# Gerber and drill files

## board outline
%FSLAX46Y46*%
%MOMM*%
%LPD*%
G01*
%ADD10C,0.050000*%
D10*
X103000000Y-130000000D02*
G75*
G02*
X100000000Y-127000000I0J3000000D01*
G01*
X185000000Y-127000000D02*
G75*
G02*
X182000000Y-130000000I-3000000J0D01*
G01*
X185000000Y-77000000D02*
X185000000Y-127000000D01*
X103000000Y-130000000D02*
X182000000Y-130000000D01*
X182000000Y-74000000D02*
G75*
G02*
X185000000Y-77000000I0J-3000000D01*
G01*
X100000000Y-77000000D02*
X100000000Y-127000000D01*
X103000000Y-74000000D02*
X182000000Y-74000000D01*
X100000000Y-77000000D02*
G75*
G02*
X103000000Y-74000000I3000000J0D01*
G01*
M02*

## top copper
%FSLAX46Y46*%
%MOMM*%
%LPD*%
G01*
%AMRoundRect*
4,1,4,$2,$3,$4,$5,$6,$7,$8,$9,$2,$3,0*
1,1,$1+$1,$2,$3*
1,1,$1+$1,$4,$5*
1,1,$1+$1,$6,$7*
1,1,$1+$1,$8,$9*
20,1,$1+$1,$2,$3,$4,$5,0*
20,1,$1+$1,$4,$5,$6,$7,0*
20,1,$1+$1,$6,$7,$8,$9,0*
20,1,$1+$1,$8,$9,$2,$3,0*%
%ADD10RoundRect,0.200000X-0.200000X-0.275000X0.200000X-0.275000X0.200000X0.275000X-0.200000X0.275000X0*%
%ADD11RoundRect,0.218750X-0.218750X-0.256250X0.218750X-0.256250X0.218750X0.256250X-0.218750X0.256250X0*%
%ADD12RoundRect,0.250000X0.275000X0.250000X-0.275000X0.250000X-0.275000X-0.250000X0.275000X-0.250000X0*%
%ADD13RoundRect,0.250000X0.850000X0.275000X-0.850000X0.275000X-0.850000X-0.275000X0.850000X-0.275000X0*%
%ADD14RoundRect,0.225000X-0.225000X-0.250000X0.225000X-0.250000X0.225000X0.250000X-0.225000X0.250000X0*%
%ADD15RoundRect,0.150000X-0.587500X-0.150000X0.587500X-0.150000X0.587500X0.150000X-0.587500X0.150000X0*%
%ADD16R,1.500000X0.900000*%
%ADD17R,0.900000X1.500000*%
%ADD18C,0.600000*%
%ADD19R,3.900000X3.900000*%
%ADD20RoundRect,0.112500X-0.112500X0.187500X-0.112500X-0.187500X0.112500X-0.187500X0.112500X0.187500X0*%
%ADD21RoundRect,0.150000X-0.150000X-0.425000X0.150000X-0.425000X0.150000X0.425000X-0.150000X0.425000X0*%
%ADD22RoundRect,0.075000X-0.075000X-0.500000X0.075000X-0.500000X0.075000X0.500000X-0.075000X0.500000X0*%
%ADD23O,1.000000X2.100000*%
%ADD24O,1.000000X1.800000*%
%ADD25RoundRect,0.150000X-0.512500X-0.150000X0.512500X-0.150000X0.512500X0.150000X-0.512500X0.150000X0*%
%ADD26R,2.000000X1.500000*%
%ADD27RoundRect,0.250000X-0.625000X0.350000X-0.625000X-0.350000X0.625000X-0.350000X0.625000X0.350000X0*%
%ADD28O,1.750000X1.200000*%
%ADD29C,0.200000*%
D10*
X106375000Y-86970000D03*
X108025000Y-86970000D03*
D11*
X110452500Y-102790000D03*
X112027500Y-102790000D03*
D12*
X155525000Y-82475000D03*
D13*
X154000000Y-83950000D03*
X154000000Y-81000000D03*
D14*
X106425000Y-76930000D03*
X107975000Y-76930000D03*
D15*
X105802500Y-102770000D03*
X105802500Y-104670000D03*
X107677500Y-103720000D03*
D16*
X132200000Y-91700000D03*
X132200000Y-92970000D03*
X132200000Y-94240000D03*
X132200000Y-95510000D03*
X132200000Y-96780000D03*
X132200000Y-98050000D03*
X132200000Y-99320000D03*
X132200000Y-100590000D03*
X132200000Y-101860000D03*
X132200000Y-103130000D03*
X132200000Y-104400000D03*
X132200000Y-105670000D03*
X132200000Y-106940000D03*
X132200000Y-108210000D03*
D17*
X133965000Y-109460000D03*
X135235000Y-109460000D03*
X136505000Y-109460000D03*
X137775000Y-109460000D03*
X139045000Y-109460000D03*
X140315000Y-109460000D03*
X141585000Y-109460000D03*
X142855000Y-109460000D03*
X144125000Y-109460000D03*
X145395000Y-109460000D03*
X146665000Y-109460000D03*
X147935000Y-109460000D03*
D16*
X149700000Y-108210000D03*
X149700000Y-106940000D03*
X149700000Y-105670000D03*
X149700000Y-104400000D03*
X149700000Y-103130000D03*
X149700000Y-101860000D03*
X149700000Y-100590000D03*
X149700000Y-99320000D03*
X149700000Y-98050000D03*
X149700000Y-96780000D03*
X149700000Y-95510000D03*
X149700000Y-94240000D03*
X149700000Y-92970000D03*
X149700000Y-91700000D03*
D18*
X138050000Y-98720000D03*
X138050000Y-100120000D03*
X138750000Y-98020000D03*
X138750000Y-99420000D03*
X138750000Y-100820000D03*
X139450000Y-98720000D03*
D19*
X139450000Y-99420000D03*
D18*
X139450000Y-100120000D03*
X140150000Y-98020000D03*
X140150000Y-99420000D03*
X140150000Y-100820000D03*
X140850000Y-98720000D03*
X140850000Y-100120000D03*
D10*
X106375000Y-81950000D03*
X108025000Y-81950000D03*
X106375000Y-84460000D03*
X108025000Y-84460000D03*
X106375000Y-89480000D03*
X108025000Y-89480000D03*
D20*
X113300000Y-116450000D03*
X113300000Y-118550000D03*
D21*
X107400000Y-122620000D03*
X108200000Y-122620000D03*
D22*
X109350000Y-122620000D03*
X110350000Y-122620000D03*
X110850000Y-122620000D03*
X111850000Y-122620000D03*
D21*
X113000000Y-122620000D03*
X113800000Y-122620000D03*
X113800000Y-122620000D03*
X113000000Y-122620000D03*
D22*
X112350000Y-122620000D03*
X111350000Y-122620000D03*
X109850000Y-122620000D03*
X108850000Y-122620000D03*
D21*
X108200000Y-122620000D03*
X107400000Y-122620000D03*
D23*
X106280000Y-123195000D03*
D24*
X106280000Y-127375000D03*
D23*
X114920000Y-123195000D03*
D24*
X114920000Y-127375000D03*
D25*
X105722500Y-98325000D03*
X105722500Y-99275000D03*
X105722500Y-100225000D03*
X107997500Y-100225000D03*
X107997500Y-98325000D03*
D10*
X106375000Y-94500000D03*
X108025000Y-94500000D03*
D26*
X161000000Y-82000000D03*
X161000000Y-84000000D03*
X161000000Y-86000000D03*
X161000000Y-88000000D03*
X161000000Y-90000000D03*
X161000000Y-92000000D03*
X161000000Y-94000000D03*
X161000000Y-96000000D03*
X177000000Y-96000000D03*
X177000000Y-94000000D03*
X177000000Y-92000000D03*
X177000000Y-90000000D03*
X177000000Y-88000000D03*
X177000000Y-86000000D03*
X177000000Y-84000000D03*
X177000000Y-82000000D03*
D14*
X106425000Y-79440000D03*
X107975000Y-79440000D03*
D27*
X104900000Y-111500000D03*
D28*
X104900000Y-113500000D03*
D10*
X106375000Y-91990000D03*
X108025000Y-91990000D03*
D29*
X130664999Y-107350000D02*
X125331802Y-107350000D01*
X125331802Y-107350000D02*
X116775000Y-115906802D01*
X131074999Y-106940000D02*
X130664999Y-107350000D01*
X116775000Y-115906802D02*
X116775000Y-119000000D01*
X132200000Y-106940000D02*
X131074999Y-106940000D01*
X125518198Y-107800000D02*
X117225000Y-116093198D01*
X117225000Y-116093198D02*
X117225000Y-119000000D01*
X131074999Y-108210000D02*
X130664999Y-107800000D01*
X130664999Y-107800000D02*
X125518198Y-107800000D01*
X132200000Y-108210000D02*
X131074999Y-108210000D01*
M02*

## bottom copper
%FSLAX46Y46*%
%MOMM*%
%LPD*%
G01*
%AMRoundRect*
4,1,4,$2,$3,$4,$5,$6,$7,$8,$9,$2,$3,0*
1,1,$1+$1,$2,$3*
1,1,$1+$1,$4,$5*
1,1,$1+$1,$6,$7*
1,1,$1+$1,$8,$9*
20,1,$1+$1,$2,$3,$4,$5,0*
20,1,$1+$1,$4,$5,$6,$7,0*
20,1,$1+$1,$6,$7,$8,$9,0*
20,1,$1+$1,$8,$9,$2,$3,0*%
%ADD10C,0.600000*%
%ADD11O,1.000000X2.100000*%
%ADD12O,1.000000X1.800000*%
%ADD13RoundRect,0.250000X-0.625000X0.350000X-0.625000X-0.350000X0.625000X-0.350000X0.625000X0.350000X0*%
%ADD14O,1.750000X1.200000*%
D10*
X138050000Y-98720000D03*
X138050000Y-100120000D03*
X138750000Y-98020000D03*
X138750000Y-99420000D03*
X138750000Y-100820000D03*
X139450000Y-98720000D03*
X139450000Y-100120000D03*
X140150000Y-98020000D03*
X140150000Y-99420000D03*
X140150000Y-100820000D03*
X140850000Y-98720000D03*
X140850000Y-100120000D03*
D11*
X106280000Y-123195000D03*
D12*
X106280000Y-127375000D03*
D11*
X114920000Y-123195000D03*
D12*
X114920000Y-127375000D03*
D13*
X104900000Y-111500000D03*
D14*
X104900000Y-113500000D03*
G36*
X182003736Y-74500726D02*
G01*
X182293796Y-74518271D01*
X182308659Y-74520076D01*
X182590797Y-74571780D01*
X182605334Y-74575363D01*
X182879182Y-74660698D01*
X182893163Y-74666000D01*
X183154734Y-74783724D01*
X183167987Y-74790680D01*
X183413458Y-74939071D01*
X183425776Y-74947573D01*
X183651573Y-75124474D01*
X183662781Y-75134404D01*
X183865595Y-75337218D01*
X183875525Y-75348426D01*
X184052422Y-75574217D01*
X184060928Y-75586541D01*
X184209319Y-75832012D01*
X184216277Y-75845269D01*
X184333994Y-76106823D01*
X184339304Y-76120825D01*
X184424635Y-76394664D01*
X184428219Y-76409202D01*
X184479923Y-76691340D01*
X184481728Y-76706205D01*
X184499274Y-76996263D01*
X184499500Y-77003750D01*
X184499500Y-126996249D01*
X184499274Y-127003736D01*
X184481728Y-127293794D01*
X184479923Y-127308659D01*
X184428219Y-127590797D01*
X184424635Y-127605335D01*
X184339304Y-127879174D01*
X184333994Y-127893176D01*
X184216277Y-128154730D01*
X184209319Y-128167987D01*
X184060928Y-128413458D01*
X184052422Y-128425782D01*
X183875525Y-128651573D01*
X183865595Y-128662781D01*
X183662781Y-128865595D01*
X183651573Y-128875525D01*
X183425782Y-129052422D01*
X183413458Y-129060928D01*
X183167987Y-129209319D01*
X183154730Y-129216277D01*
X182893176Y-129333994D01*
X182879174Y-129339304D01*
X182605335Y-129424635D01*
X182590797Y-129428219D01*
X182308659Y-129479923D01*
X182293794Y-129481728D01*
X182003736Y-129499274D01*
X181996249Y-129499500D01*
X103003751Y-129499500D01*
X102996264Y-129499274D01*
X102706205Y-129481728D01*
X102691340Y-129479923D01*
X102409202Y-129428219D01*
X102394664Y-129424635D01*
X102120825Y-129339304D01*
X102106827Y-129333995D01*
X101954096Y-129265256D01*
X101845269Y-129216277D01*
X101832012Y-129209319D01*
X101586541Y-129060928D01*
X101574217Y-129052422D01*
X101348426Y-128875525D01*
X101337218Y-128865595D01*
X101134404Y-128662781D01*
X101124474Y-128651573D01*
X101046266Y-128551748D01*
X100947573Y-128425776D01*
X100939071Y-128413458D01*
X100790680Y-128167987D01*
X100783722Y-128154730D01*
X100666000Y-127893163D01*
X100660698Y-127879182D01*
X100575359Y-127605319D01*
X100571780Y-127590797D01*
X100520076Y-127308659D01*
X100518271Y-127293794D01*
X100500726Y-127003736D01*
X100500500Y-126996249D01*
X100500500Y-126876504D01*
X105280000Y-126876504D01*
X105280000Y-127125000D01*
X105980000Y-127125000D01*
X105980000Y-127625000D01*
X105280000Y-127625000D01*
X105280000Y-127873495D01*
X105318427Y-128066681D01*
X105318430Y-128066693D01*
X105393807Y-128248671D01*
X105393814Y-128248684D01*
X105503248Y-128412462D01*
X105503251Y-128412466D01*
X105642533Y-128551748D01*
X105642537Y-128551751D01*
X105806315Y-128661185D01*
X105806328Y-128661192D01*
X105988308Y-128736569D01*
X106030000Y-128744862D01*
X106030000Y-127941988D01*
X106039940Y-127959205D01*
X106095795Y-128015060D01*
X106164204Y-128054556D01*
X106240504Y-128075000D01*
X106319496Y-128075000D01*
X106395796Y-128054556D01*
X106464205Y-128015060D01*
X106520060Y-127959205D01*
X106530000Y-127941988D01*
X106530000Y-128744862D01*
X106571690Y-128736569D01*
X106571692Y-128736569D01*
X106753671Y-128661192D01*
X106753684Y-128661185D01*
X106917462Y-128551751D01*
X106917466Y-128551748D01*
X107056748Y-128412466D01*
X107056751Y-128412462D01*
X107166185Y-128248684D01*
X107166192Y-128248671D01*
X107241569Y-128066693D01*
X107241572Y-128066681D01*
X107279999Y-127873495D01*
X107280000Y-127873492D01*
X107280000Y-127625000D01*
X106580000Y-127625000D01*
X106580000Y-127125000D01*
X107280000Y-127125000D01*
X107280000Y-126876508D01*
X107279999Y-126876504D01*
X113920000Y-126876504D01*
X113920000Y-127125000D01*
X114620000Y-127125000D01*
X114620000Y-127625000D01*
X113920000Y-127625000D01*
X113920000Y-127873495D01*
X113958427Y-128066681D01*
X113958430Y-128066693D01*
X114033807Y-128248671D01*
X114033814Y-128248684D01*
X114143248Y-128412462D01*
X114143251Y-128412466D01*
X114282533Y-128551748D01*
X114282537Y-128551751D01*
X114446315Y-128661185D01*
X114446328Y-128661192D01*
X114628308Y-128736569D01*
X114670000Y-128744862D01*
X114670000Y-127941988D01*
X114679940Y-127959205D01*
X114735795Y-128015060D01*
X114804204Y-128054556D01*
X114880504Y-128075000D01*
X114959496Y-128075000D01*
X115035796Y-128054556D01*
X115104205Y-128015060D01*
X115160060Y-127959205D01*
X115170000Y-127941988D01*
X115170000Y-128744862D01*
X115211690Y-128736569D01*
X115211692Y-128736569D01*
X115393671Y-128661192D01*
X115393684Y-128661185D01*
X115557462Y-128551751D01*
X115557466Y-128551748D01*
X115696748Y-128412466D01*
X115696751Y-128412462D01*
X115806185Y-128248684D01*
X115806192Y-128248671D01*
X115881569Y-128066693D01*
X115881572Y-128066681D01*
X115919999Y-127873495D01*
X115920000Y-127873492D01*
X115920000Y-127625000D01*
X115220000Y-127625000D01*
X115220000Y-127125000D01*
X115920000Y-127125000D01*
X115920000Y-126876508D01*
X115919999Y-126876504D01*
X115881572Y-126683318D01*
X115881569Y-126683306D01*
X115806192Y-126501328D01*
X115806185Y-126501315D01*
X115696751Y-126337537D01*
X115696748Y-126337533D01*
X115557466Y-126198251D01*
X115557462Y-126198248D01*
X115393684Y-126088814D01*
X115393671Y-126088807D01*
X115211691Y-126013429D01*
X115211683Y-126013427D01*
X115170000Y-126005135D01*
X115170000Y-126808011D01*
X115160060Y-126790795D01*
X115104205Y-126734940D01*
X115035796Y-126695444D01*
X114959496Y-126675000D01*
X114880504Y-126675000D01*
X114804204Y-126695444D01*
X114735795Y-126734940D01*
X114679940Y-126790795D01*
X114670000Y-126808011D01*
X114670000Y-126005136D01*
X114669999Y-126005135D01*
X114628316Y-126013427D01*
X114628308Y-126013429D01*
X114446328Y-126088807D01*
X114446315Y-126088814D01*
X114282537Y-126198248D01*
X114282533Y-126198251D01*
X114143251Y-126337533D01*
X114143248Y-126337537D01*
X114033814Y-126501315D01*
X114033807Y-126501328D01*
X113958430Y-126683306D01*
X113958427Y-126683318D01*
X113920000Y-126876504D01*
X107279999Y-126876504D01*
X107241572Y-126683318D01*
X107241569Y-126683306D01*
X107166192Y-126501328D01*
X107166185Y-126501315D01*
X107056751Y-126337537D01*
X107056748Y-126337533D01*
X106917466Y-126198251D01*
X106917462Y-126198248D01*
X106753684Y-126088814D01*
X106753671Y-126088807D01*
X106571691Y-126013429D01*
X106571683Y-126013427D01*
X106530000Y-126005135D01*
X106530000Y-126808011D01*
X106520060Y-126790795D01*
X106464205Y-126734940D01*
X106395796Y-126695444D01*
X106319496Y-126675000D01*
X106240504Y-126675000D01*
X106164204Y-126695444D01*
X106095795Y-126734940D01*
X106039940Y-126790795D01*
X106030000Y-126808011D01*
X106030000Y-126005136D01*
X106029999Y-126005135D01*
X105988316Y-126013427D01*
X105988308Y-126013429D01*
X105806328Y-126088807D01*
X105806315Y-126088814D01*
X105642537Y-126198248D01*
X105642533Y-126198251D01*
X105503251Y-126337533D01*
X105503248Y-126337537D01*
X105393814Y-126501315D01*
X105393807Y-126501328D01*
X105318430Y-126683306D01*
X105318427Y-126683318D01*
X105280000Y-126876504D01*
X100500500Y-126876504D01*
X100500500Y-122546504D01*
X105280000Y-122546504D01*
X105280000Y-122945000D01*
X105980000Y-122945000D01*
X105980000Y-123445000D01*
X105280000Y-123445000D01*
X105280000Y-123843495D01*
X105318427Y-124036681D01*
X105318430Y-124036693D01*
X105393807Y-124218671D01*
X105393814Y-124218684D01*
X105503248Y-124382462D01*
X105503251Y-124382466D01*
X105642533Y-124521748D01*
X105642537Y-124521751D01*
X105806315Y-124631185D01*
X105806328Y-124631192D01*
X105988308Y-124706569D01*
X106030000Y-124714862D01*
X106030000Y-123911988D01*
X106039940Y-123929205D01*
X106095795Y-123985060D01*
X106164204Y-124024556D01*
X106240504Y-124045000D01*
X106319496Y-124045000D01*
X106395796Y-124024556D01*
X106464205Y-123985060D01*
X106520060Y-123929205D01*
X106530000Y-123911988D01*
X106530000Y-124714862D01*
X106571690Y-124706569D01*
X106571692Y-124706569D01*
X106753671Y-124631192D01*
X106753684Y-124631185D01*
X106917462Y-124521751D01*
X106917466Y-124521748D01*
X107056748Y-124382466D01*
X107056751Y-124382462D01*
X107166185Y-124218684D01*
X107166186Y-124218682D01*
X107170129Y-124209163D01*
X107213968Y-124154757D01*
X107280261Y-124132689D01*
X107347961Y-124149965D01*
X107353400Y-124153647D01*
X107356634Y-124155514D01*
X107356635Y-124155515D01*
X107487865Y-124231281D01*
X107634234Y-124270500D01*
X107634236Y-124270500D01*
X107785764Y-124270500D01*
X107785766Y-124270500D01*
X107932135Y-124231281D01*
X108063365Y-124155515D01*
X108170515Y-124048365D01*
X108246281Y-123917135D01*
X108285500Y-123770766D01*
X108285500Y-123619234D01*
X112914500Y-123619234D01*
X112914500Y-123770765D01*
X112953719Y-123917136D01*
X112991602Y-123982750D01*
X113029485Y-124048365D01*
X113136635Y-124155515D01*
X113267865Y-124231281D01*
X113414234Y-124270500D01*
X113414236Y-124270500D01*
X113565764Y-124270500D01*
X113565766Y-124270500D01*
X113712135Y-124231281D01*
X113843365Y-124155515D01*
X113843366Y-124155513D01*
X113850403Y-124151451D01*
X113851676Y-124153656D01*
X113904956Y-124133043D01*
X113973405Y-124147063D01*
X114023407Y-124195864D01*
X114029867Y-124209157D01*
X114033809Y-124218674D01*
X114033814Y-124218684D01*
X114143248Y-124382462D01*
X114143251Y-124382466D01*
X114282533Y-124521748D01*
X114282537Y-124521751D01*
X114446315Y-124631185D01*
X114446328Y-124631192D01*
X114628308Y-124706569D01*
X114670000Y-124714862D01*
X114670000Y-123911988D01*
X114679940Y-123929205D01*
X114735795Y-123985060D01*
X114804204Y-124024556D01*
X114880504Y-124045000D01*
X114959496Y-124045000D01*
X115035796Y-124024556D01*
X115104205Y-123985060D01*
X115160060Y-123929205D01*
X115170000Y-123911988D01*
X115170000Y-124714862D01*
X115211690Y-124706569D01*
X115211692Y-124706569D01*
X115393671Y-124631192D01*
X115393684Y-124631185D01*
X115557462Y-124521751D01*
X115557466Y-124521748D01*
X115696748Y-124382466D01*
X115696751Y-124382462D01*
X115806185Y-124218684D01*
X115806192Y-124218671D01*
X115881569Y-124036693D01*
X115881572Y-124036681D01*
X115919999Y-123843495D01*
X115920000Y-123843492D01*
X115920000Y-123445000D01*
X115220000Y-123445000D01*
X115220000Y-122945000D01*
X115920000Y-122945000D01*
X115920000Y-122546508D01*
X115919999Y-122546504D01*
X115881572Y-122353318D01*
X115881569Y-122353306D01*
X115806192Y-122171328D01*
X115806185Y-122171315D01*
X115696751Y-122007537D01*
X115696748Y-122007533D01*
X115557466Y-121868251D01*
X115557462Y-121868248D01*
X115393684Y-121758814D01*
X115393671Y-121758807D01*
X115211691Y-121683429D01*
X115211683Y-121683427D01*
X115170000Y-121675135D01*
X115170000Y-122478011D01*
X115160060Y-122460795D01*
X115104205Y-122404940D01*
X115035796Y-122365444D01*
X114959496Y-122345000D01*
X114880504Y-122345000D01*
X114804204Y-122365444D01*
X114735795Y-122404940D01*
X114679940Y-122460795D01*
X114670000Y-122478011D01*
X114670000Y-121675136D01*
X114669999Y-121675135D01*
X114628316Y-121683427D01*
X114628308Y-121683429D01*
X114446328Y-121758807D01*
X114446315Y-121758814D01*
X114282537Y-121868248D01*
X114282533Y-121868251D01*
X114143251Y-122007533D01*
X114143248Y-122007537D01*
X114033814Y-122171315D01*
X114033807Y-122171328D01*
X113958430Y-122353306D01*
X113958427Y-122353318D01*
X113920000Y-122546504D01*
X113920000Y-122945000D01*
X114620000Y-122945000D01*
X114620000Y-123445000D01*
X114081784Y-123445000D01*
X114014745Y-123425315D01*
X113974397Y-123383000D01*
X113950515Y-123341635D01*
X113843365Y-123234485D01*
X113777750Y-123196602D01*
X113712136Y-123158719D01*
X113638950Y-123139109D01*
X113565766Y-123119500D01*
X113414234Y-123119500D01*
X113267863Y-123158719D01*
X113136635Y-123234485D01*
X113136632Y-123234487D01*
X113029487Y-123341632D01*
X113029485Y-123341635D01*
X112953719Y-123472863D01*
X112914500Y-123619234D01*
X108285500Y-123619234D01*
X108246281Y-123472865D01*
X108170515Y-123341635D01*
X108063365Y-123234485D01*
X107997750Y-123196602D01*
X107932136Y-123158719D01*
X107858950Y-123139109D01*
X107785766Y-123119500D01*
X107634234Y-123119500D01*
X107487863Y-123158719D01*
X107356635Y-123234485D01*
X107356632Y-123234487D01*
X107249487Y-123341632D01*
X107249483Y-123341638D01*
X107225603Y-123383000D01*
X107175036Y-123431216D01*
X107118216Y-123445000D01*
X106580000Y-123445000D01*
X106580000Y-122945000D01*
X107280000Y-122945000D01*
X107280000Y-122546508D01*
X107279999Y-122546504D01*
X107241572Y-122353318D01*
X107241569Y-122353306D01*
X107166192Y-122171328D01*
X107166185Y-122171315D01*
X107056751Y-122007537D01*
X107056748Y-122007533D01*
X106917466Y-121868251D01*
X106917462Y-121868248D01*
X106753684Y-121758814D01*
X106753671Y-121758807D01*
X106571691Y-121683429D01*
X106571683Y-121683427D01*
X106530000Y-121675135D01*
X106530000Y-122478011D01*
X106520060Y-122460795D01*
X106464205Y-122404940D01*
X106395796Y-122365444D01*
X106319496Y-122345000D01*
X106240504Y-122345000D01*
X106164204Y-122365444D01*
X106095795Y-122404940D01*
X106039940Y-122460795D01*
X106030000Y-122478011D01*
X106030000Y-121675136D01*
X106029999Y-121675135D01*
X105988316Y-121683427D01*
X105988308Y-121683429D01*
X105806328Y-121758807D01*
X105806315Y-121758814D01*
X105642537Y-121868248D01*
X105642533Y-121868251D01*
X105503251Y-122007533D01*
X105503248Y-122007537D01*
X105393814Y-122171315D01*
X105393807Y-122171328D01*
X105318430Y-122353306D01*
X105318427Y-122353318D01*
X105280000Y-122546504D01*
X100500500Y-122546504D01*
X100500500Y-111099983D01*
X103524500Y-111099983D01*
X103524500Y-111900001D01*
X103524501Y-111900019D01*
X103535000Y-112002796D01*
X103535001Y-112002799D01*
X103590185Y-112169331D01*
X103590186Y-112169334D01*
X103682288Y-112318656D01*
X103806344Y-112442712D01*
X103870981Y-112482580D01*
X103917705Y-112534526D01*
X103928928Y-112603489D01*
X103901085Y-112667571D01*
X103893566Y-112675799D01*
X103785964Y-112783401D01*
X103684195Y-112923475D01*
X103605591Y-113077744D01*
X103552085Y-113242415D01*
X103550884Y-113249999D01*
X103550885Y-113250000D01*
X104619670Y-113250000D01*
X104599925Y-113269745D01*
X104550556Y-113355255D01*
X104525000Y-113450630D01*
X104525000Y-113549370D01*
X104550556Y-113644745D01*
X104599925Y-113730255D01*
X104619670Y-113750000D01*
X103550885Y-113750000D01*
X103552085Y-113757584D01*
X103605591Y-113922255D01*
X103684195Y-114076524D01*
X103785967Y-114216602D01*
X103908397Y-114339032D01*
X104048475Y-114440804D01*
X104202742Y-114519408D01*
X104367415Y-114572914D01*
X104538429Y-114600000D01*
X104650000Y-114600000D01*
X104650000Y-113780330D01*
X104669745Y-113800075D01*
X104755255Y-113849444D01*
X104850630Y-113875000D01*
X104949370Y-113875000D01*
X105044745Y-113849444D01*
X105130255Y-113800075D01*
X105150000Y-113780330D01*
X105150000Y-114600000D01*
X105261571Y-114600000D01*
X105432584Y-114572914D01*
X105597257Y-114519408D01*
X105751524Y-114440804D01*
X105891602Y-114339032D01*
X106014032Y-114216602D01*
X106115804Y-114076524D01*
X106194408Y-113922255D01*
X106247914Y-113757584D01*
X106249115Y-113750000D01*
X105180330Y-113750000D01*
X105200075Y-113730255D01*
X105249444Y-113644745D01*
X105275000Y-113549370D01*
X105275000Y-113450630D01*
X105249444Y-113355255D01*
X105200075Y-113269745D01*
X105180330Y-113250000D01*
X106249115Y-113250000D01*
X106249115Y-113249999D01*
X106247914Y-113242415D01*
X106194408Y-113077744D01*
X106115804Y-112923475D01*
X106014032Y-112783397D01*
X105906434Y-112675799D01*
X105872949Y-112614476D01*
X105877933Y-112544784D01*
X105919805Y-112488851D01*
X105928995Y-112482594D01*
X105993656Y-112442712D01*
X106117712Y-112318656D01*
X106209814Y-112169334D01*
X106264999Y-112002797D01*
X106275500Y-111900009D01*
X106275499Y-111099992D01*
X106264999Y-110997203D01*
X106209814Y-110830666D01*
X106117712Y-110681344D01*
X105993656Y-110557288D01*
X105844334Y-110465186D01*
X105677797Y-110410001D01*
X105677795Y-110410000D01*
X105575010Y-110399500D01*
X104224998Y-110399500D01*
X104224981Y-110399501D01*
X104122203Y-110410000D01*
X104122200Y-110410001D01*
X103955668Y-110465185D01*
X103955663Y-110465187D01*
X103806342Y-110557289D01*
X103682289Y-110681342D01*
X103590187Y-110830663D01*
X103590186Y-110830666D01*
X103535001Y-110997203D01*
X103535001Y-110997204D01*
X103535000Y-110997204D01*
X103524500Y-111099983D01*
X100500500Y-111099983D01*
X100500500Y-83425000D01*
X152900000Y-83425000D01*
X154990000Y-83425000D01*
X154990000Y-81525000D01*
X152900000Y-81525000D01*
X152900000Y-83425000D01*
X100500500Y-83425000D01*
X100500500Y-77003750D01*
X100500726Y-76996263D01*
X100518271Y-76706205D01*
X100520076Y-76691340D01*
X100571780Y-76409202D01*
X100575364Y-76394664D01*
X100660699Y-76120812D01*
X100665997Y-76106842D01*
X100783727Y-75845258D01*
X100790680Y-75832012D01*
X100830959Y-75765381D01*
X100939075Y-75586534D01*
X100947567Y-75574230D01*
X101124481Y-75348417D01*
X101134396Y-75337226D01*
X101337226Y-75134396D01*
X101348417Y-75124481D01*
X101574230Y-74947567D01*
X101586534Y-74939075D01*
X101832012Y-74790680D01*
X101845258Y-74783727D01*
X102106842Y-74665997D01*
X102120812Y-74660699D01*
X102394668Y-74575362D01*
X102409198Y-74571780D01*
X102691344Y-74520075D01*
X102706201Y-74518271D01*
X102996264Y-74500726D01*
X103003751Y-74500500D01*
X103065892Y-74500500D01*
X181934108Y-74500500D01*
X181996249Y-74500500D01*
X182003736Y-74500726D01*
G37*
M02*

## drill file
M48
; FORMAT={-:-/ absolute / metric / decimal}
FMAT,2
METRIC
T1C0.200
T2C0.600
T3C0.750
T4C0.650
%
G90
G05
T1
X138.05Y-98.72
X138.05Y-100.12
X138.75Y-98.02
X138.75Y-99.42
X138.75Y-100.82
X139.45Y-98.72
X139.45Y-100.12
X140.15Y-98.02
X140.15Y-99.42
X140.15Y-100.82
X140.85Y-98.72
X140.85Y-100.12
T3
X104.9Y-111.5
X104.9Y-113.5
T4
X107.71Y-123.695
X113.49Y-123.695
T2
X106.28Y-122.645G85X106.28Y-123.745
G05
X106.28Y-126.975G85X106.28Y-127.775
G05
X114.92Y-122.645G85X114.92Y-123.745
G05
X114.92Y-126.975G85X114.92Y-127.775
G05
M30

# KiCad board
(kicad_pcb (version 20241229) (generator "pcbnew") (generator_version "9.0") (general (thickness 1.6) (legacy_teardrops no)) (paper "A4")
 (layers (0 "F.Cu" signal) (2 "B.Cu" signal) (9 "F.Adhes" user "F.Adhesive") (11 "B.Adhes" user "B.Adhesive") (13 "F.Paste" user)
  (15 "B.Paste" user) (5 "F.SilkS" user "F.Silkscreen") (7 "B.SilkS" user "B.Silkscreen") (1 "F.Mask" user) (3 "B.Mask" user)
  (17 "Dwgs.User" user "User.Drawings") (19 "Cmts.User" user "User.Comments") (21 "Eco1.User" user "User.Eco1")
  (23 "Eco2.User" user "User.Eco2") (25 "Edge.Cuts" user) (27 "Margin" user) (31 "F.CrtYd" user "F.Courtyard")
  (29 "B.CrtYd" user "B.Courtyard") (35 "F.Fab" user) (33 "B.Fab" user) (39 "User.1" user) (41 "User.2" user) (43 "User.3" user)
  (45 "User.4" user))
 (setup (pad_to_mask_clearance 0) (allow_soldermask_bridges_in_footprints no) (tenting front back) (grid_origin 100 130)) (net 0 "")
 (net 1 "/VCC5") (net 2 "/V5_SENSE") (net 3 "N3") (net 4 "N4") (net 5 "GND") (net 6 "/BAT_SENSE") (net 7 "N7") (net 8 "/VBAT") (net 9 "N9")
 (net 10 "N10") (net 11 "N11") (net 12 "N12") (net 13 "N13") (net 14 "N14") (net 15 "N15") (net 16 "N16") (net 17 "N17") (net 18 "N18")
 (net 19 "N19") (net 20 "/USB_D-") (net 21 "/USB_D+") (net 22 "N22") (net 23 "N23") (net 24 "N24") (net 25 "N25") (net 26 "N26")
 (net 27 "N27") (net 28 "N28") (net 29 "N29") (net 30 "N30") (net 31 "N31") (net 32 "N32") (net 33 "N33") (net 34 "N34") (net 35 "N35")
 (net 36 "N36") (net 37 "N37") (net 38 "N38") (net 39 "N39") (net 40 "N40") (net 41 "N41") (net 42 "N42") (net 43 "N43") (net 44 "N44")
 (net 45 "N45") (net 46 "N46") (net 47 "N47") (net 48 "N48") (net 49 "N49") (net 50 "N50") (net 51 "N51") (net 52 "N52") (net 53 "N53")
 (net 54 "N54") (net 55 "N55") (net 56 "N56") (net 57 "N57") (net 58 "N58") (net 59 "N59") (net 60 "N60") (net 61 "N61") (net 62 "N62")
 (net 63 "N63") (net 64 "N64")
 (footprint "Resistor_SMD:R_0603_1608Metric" (layer "F.Cu") (at 107.2 86.97)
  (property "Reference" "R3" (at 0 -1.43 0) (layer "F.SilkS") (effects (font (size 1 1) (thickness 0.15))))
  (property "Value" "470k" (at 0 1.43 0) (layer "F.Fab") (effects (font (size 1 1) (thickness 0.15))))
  (pad "1" smd roundrect (at -0.825 0) (size 0.8 0.95) (layers "F.Cu" "F.Mask" "F.Paste") (roundrect_rratio 0.25) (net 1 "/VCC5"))
  (pad "2" smd roundrect (at 0.825 0) (size 0.8 0.95) (layers "F.Cu" "F.Mask" "F.Paste") (roundrect_rratio 0.25) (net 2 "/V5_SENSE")))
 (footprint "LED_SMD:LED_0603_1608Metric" (layer "F.Cu") (at 111.24 102.79)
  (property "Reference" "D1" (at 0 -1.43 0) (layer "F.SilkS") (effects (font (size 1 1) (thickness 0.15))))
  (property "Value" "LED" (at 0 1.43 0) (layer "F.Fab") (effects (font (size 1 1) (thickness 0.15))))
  (pad "1" smd roundrect (at -0.7875 0) (size 0.875 0.95) (layers "F.Cu" "F.Mask" "F.Paste") (roundrect_rratio 0.25) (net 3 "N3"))
  (pad "2" smd roundrect (at 0.7875 0) (size 0.875 0.95) (layers "F.Cu" "F.Mask" "F.Paste") (roundrect_rratio 0.25) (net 1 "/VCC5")))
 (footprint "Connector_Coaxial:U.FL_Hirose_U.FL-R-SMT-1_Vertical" (layer "F.Cu") (at 154.475 82.475 180)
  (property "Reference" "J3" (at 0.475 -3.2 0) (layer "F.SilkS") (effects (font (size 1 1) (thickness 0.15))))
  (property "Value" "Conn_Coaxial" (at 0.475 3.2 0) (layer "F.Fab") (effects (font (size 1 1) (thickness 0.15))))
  (pad "1" smd roundrect (at -1.05 0 180) (size 1.05 1) (layers "F.Cu" "F.Mask" "F.Paste") (roundrect_rratio 0.25) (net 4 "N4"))
  (pad "2" smd roundrect (at 0.475 -1.475 180) (size 2.2 1.05) (layers "F.Cu" "F.Mask" "F.Paste") (roundrect_rratio 0.2380952381)
   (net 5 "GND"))
  (pad "2" smd roundrect (at 0.475 1.475 180) (size 2.2 1.05) (layers "F.Cu" "F.Mask" "F.Paste") (roundrect_rratio 0.2380952381)
   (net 5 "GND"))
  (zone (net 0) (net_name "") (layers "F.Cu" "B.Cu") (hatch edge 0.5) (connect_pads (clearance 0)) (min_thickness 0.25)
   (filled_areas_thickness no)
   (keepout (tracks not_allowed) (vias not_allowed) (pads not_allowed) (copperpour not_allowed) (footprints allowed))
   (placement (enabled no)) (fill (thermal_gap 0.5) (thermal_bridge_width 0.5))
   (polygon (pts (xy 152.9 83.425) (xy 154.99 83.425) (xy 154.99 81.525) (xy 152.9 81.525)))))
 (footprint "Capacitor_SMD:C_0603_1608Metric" (layer "F.Cu") (at 107.2 76.93)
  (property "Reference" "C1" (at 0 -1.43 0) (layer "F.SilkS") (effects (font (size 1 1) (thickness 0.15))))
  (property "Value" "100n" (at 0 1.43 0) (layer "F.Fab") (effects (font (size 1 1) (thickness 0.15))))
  (pad "1" smd roundrect (at -0.775 0) (size 0.9 0.95) (layers "F.Cu" "F.Mask" "F.Paste") (roundrect_rratio 0.25) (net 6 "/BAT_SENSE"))
  (pad "2" smd roundrect (at 0.775 0) (size 0.9 0.95) (layers "F.Cu" "F.Mask" "F.Paste") (roundrect_rratio 0.25) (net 5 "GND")))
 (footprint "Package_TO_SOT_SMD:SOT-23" (layer "F.Cu") (at 106.74 103.72)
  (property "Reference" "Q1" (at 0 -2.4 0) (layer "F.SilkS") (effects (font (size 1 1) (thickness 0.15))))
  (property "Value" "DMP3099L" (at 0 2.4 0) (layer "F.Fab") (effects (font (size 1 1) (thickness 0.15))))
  (pad "1" smd roundrect (at -0.9375 -0.95) (size 1.475 0.6) (layers "F.Cu" "F.Mask" "F.Paste") (roundrect_rratio 0.25) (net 1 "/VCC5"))
  (pad "2" smd roundrect (at -0.9375 0.95) (size 1.475 0.6) (layers "F.Cu" "F.Mask" "F.Paste") (roundrect_rratio 0.25) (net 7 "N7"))
  (pad "3" smd roundrect (at 0.9375 0) (size 1.475 0.6) (layers "F.Cu" "F.Mask" "F.Paste") (roundrect_rratio 0.25) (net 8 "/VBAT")))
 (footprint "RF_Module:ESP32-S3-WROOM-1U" (layer "F.Cu") (at 140.95 100.11)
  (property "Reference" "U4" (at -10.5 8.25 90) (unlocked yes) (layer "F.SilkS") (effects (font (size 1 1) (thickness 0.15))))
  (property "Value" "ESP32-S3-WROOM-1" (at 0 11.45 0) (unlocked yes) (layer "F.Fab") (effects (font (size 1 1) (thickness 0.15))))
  (pad "" smd rect (at -2.904394 0.71) (size 0.9 0.9) (layers "F.Paste"))
  (pad "" smd rect (at -2.9 -2.09) (size 0.9 0.9) (layers "F.Paste"))
  (pad "" smd rect (at -2.9 -0.69) (size 0.9 0.9) (layers "F.Paste"))
  (pad "" smd rect (at -1.504394 0.71) (size 0.9 0.9) (layers "F.Paste"))
  (pad "" smd rect (at -1.5 -2.09) (size 0.9 0.9) (layers "F.Paste"))
  (pad "" smd rect (at -1.5 -0.69) (size 0.9 0.9) (layers "F.Paste"))
  (pad "" smd rect (at -0.104394 0.71) (size 0.9 0.9) (layers "F.Paste"))
  (pad "" smd rect (at -0.1 -2.09) (size 0.9 0.9) (layers "F.Paste"))
  (pad "" smd rect (at -0.1 -0.69) (size 0.9 0.9) (layers "F.Paste"))
  (pad "1" smd rect (at -8.75 -8.41) (size 1.5 0.9) (layers "F.Cu" "F.Mask" "F.Paste") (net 5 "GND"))
  (pad "2" smd rect (at -8.75 -7.14) (size 1.5 0.9) (layers "F.Cu" "F.Mask" "F.Paste") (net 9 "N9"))
  (pad "3" smd rect (at -8.75 -5.87) (size 1.5 0.9) (layers "F.Cu" "F.Mask" "F.Paste") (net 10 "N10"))
  (pad "4" smd rect (at -8.75 -4.6) (size 1.5 0.9) (layers "F.Cu" "F.Mask" "F.Paste") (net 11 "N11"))
  (pad "5" smd rect (at -8.75 -3.33) (size 1.5 0.9) (layers "F.Cu" "F.Mask" "F.Paste") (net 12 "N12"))
  (pad "6" smd rect (at -8.75 -2.06) (size 1.5 0.9) (layers "F.Cu" "F.Mask" "F.Paste") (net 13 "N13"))
  (pad "7" smd rect (at -8.75 -0.79) (size 1.5 0.9) (layers "F.Cu" "F.Mask" "F.Paste") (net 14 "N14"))
  (pad "8" smd rect (at -8.75 0.48) (size 1.5 0.9) (layers "F.Cu" "F.Mask" "F.Paste") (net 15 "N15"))
  (pad "9" smd rect (at -8.75 1.75) (size 1.5 0.9) (layers "F.Cu" "F.Mask" "F.Paste") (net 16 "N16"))
  (pad "10" smd rect (at -8.75 3.02) (size 1.5 0.9) (layers "F.Cu" "F.Mask" "F.Paste") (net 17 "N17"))
  (pad "11" smd rect (at -8.75 4.29) (size 1.5 0.9) (layers "F.Cu" "F.Mask" "F.Paste") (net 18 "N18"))
  (pad "12" smd rect (at -8.75 5.56) (size 1.5 0.9) (layers "F.Cu" "F.Mask" "F.Paste") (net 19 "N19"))
  (pad "13" smd rect (at -8.75 6.83) (size 1.5 0.9) (layers "F.Cu" "F.Mask" "F.Paste") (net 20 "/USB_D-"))
  (pad "14" smd rect (at -8.75 8.1 180) (size 1.5 0.9) (layers "F.Cu" "F.Mask" "F.Paste") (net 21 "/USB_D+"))
  (pad "15" smd rect (at -6.985 9.35 270) (size 1.5 0.9) (layers "F.Cu" "F.Mask" "F.Paste") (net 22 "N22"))
  (pad "16" smd rect (at -5.715 9.35 270) (size 1.5 0.9) (layers "F.Cu" "F.Mask" "F.Paste") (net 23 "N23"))
  (pad "17" smd rect (at -4.445 9.35 270) (size 1.5 0.9) (layers "F.Cu" "F.Mask" "F.Paste") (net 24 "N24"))
  (pad "18" smd rect (at -3.175 9.35 270) (size 1.5 0.9) (layers "F.Cu" "F.Mask" "F.Paste") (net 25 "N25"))
  (pad "19" smd rect (at -1.905 9.35 270) (size 1.5 0.9) (layers "F.Cu" "F.Mask" "F.Paste") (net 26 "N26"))
  (pad "20" smd rect (at -0.635 9.35 270) (size 1.5 0.9) (layers "F.Cu" "F.Mask" "F.Paste") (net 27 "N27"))
  (pad "21" smd rect (at 0.635 9.35 270) (size 1.5 0.9) (layers "F.Cu" "F.Mask" "F.Paste") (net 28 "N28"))
  (pad "22" smd rect (at 1.905 9.35 270) (size 1.5 0.9) (layers "F.Cu" "F.Mask" "F.Paste") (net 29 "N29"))
  (pad "23" smd rect (at 3.175 9.35 270) (size 1.5 0.9) (layers "F.Cu" "F.Mask" "F.Paste") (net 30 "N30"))
  (pad "24" smd rect (at 4.445 9.35 270) (size 1.5 0.9) (layers "F.Cu" "F.Mask" "F.Paste") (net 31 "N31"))
  (pad "25" smd rect (at 5.715 9.35 270) (size 1.5 0.9) (layers "F.Cu" "F.Mask" "F.Paste") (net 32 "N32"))
  (pad "26" smd rect (at 6.985 9.35 270) (size 1.5 0.9) (layers "F.Cu" "F.Mask" "F.Paste") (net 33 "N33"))
  (pad "27" smd rect (at 8.75 8.1) (size 1.5 0.9) (layers "F.Cu" "F.Mask" "F.Paste") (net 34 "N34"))
  (pad "28" smd rect (at 8.75 6.83) (size 1.5 0.9) (layers "F.Cu" "F.Mask" "F.Paste") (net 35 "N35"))
  (pad "29" smd rect (at 8.75 5.56) (size 1.5 0.9) (layers "F.Cu" "F.Mask" "F.Paste") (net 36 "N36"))
  (pad "30" smd rect (at 8.75 4.29) (size 1.5 0.9) (layers "F.Cu" "F.Mask" "F.Paste") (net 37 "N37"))
  (pad "31" smd rect (at 8.75 3.02) (size 1.5 0.9) (layers "F.Cu" "F.Mask" "F.Paste") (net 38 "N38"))
  (pad "32" smd rect (at 8.75 1.75) (size 1.5 0.9) (layers "F.Cu" "F.Mask" "F.Paste") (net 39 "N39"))
  (pad "33" smd rect (at 8.75 0.48) (size 1.5 0.9) (layers "F.Cu" "F.Mask" "F.Paste") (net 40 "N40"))
  (pad "34" smd rect (at 8.75 -0.79) (size 1.5 0.9) (layers "F.Cu" "F.Mask" "F.Paste") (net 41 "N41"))
  (pad "35" smd rect (at 8.75 -2.06) (size 1.5 0.9) (layers "F.Cu" "F.Mask" "F.Paste") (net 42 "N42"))
  (pad "36" smd rect (at 8.75 -3.33) (size 1.5 0.9) (layers "F.Cu" "F.Mask" "F.Paste") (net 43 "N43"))
  (pad "37" smd rect (at 8.75 -4.6) (size 1.5 0.9) (layers "F.Cu" "F.Mask" "F.Paste") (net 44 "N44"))
  (pad "38" smd rect (at 8.75 -5.87) (size 1.5 0.9) (layers "F.Cu" "F.Mask" "F.Paste") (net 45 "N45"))
  (pad "39" smd rect (at 8.75 -7.14) (size 1.5 0.9) (layers "F.Cu" "F.Mask" "F.Paste") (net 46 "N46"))
  (pad "40" smd rect (at 8.75 -8.41) (size 1.5 0.9) (layers "F.Cu" "F.Mask" "F.Paste") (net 5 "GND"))
  (pad "41" thru_hole circle (at -2.9 -1.39) (size 0.6 0.6) (drill 0.2) (layers "*.Cu" "F.Mask") (remove_unused_layers no) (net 5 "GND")
   (zone_connect 2))
  (pad "41" thru_hole circle (at -2.9 0.01) (size 0.6 0.6) (drill 0.2) (layers "*.Cu" "F.Mask") (remove_unused_layers no) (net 5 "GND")
   (zone_connect 2))
  (pad "41" thru_hole circle (at -2.2 -2.09) (size 0.6 0.6) (drill 0.2) (layers "*.Cu" "F.Mask") (remove_unused_layers no) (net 5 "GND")
   (zone_connect 2))
  (pad "41" thru_hole circle (at -2.2 -0.69) (size 0.6 0.6) (drill 0.2) (layers "*.Cu" "F.Mask") (remove_unused_layers no) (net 5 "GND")
   (zone_connect 2))
  (pad "41" thru_hole circle (at -2.2 0.71) (size 0.6 0.6) (drill 0.2) (layers "*.Cu" "F.Mask") (remove_unused_layers no) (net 5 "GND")
   (zone_connect 2))
  (pad "41" thru_hole circle (at -1.5 -1.39) (size 0.6 0.6) (drill 0.2) (layers "*.Cu" "F.Mask") (remove_unused_layers no) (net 5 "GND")
   (zone_connect 2))
  (pad "41" smd rect (at -1.5 -0.69) (size 3.9 3.9) (layers "F.Cu" "F.Mask") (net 5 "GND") (zone_connect 2))
  (pad "41" thru_hole circle (at -1.5 0.01) (size 0.6 0.6) (drill 0.2) (layers "*.Cu" "F.Mask") (remove_unused_layers no) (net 5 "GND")
   (zone_connect 2))
  (pad "41" thru_hole circle (at -0.8 -2.09) (size 0.6 0.6) (drill 0.2) (layers "*.Cu" "F.Mask") (remove_unused_layers no) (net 5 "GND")
   (zone_connect 2))
  (pad "41" thru_hole circle (at -0.8 -0.69) (size 0.6 0.6) (drill 0.2) (layers "*.Cu" "F.Mask") (remove_unused_layers no) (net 5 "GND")
   (zone_connect 2))
  (pad "41" thru_hole circle (at -0.8 0.71) (size 0.6 0.6) (drill 0.2) (layers "*.Cu" "F.Mask") (remove_unused_layers no) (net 5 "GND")
   (zone_connect 2))
  (pad "41" thru_hole circle (at -0.1 -1.39) (size 0.6 0.6) (drill 0.2) (layers "*.Cu" "F.Mask") (remove_unused_layers no) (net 5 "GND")
   (zone_connect 2))
  (pad "41" thru_hole circle (at -0.1 0.01) (size 0.6 0.6) (drill 0.2) (layers "*.Cu" "F.Mask") (remove_unused_layers no) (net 5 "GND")
   (zone_connect 2)))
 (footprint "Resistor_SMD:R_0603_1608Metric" (layer "F.Cu") (at 107.2 81.95)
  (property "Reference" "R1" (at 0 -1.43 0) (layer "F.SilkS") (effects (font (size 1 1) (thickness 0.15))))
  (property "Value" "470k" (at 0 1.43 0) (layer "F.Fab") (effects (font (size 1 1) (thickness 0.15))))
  (pad "1" smd roundrect (at -0.825 0) (size 0.8 0.95) (layers "F.Cu" "F.Mask" "F.Paste") (roundrect_rratio 0.25) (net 8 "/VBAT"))
  (pad "2" smd roundrect (at 0.825 0) (size 0.8 0.95) (layers "F.Cu" "F.Mask" "F.Paste") (roundrect_rratio 0.25) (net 6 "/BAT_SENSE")))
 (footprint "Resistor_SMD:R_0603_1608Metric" (layer "F.Cu") (at 107.2 84.46)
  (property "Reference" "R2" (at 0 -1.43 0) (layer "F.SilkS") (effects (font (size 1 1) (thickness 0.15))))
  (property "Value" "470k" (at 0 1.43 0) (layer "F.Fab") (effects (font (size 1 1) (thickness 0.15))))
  (pad "1" smd roundrect (at -0.825 0) (size 0.8 0.95) (layers "F.Cu" "F.Mask" "F.Paste") (roundrect_rratio 0.25) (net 6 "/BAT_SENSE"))
  (pad "2" smd roundrect (at 0.825 0) (size 0.8 0.95) (layers "F.Cu" "F.Mask" "F.Paste") (roundrect_rratio 0.25) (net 5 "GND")))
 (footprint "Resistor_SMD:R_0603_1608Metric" (layer "F.Cu") (at 107.2 89.48)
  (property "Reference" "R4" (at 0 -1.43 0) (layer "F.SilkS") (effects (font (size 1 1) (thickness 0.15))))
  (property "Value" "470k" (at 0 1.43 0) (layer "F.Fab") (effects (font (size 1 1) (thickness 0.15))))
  (pad "1" smd roundrect (at -0.825 0) (size 0.8 0.95) (layers "F.Cu" "F.Mask" "F.Paste") (roundrect_rratio 0.25) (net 2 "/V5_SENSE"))
  (pad "2" smd roundrect (at 0.825 0) (size 0.8 0.95) (layers "F.Cu" "F.Mask" "F.Paste") (roundrect_rratio 0.25) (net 5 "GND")))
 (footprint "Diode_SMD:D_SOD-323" (layer "F.Cu") (at 113.3 117.5 -90)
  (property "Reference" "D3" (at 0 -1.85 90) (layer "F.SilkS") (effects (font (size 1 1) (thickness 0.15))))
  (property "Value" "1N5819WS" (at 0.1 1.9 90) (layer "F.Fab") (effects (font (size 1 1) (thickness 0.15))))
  (pad "1" smd roundrect (at -1.05 0 270) (size 0.6 0.45) (layers "F.Cu" "F.Mask" "F.Paste") (roundrect_rratio 0.25) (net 7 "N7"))
  (pad "2" smd roundrect (at 1.05 0 270) (size 0.6 0.45) (layers "F.Cu" "F.Mask" "F.Paste") (roundrect_rratio 0.25) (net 1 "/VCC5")))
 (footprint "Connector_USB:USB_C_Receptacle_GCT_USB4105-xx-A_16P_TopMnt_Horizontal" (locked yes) (layer "F.Cu") (at 110.6 126.3)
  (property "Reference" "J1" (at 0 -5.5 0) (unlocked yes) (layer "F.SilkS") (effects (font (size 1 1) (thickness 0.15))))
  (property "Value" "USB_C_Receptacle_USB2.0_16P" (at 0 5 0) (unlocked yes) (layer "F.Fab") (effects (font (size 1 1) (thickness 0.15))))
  (pad "" np_thru_hole circle (at -2.89 -2.605) (size 0.65 0.65) (drill 0.65) (layers "*.Cu" "*.Mask"))
  (pad "" np_thru_hole circle (at 2.89 -2.605) (size 0.65 0.65) (drill 0.65) (layers "*.Cu" "*.Mask"))
  (pad "A1" smd roundrect (at -3.2 -3.68) (size 0.6 1.15) (layers "F.Cu" "F.Mask" "F.Paste") (roundrect_rratio 0.25) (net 5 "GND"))
  (pad "A4" smd roundrect (at -2.4 -3.68) (size 0.6 1.15) (layers "F.Cu" "F.Mask" "F.Paste") (roundrect_rratio 0.25) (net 1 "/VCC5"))
  (pad "A5" smd roundrect (at -1.25 -3.68) (size 0.3 1.15) (layers "F.Cu" "F.Mask" "F.Paste") (roundrect_rratio 0.25) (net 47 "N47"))
  (pad "A6" smd roundrect (at -0.25 -3.68) (size 0.3 1.15) (layers "F.Cu" "F.Mask" "F.Paste") (roundrect_rratio 0.25) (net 21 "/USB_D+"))
  (pad "A7" smd roundrect (at 0.25 -3.68) (size 0.3 1.15) (layers "F.Cu" "F.Mask" "F.Paste") (roundrect_rratio 0.25) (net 20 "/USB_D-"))
  (pad "A8" smd roundrect (at 1.25 -3.68) (size 0.3 1.15) (layers "F.Cu" "F.Mask" "F.Paste") (roundrect_rratio 0.25) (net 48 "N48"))
  (pad "A9" smd roundrect (at 2.4 -3.68) (size 0.6 1.15) (layers "F.Cu" "F.Mask" "F.Paste") (roundrect_rratio 0.25) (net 1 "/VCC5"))
  (pad "A12" smd roundrect (at 3.2 -3.68) (size 0.6 1.15) (layers "F.Cu" "F.Mask" "F.Paste") (roundrect_rratio 0.25) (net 5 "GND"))
  (pad "B1" smd roundrect (at 3.2 -3.68) (size 0.6 1.15) (layers "F.Cu" "F.Mask" "F.Paste") (roundrect_rratio 0.25) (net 5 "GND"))
  (pad "B4" smd roundrect (at 2.4 -3.68) (size 0.6 1.15) (layers "F.Cu" "F.Mask" "F.Paste") (roundrect_rratio 0.25) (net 1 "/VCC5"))
  (pad "B5" smd roundrect (at 1.75 -3.68) (size 0.3 1.15) (layers "F.Cu" "F.Mask" "F.Paste") (roundrect_rratio 0.25) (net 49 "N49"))
  (pad "B6" smd roundrect (at 0.75 -3.68) (size 0.3 1.15) (layers "F.Cu" "F.Mask" "F.Paste") (roundrect_rratio 0.25) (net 21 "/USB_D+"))
  (pad "B7" smd roundrect (at -0.75 -3.68) (size 0.3 1.15) (layers "F.Cu" "F.Mask" "F.Paste") (roundrect_rratio 0.25) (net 20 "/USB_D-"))
  (pad "B8" smd roundrect (at -1.75 -3.68) (size 0.3 1.15) (layers "F.Cu" "F.Mask" "F.Paste") (roundrect_rratio 0.25) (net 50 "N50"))
  (pad "B9" smd roundrect (at -2.4 -3.68) (size 0.6 1.15) (layers "F.Cu" "F.Mask" "F.Paste") (roundrect_rratio 0.25) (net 1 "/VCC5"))
  (pad "B12" smd roundrect (at -3.2 -3.68) (size 0.6 1.15) (layers "F.Cu" "F.Mask" "F.Paste") (roundrect_rratio 0.25) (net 5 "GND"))
  (pad "S1" thru_hole oval (at -4.32 -3.105) (size 1 2.1) (drill oval 0.6 1.7) (layers "*.Cu" "*.Mask" "F.Paste") (remove_unused_layers no)
   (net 5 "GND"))
  (pad "S1" thru_hole oval (at -4.32 1.075) (size 1 1.8) (drill oval 0.6 1.4) (layers "*.Cu" "*.Mask" "F.Paste") (remove_unused_layers no)
   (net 5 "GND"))
  (pad "S1" thru_hole oval (at 4.32 -3.105) (size 1 2.1) (drill oval 0.6 1.7) (layers "*.Cu" "*.Mask" "F.Paste") (remove_unused_layers no)
   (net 5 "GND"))
  (pad "S1" thru_hole oval (at 4.32 1.075) (size 1 1.8) (drill oval 0.6 1.4) (layers "*.Cu" "*.Mask" "F.Paste") (remove_unused_layers no)
   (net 5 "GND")))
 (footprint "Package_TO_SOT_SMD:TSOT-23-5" (layer "F.Cu") (at 106.86 99.275)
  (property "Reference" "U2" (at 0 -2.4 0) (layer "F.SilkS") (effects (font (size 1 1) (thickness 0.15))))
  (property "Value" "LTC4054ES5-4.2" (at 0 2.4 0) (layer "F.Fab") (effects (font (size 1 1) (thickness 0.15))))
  (pad "1" smd roundrect (at -1.1375 -0.95) (size 1.325 0.6) (layers "F.Cu" "F.Mask" "F.Paste") (roundrect_rratio 0.25) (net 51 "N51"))
  (pad "2" smd roundrect (at -1.1375 0) (size 1.325 0.6) (layers "F.Cu" "F.Mask" "F.Paste") (roundrect_rratio 0.25) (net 5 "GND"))
  (pad "3" smd roundrect (at -1.1375 0.95) (size 1.325 0.6) (layers "F.Cu" "F.Mask" "F.Paste") (roundrect_rratio 0.25) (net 8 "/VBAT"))
  (pad "4" smd roundrect (at 1.1375 0.95) (size 1.325 0.6) (layers "F.Cu" "F.Mask" "F.Paste") (roundrect_rratio 0.25) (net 1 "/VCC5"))
  (pad "5" smd roundrect (at 1.1375 -0.95) (size 1.325 0.6) (layers "F.Cu" "F.Mask" "F.Paste") (roundrect_rratio 0.25) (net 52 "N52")))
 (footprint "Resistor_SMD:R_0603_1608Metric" (layer "F.Cu") (at 107.2 94.5)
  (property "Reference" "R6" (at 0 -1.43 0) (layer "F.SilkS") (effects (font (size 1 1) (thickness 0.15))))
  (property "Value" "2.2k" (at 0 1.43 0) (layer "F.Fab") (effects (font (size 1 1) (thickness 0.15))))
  (pad "1" smd roundrect (at -0.825 0) (size 0.8 0.95) (layers "F.Cu" "F.Mask" "F.Paste") (roundrect_rratio 0.25) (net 52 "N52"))
  (pad "2" smd roundrect (at 0.825 0) (size 0.8 0.95) (layers "F.Cu" "F.Mask" "F.Paste") (roundrect_rratio 0.25) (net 5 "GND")))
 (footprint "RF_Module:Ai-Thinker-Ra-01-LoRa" (layer "F.Cu") (at 169 89)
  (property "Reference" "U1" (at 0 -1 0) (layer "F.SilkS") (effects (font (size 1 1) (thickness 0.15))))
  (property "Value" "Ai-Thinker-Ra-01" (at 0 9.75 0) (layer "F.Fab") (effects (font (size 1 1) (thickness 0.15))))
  (pad "1" smd rect (at -8 -7) (size 2 1.5) (layers "F.Cu" "F.Mask" "F.Paste") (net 4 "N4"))
  (pad "2" smd rect (at -8 -5) (size 2 1.5) (layers "F.Cu" "F.Mask" "F.Paste") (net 5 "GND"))
  (pad "3" smd rect (at -8 -3) (size 2 1.5) (layers "F.Cu" "F.Mask" "F.Paste") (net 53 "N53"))
  (pad "4" smd rect (at -8 -1) (size 2 1.5) (layers "F.Cu" "F.Mask" "F.Paste") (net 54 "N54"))
  (pad "5" smd rect (at -8 1) (size 2 1.5) (layers "F.Cu" "F.Mask" "F.Paste") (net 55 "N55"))
  (pad "6" smd rect (at -8 3) (size 2 1.5) (layers "F.Cu" "F.Mask" "F.Paste") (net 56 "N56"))
  (pad "7" smd rect (at -8 5) (size 2 1.5) (layers "F.Cu" "F.Mask" "F.Paste") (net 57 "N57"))
  (pad "8" smd rect (at -8 7) (size 2 1.5) (layers "F.Cu" "F.Mask" "F.Paste") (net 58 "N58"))
  (pad "9" smd rect (at 8 7) (size 2 1.5) (layers "F.Cu" "F.Mask" "F.Paste") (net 5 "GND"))
  (pad "10" smd rect (at 8 5) (size 2 1.5) (layers "F.Cu" "F.Mask" "F.Paste") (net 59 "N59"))
  (pad "11" smd rect (at 8 3) (size 2 1.5) (layers "F.Cu" "F.Mask" "F.Paste") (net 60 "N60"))
  (pad "12" smd rect (at 8 1) (size 2 1.5) (layers "F.Cu" "F.Mask" "F.Paste") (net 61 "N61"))
  (pad "13" smd rect (at 8 -1) (size 2 1.5) (layers "F.Cu" "F.Mask" "F.Paste") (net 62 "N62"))
  (pad "14" smd rect (at 8 -3) (size 2 1.5) (layers "F.Cu" "F.Mask" "F.Paste") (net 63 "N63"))
  (pad "15" smd rect (at 8 -5) (size 2 1.5) (layers "F.Cu" "F.Mask" "F.Paste") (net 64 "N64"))
  (pad "16" smd rect (at 8 -7) (size 2 1.5) (layers "F.Cu" "F.Mask" "F.Paste") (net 5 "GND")))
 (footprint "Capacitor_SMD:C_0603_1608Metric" (layer "F.Cu") (at 107.2 79.44)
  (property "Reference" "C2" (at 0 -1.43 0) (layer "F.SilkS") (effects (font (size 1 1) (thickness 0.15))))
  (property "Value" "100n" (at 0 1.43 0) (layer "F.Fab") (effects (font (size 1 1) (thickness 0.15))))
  (pad "1" smd roundrect (at -0.775 0) (size 0.9 0.95) (layers "F.Cu" "F.Mask" "F.Paste") (roundrect_rratio 0.25) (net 2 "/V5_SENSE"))
  (pad "2" smd roundrect (at 0.775 0) (size 0.9 0.95) (layers "F.Cu" "F.Mask" "F.Paste") (roundrect_rratio 0.25) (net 5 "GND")))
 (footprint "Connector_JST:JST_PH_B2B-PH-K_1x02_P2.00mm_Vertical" (layer "F.Cu") (at 104.9 111.5 -90)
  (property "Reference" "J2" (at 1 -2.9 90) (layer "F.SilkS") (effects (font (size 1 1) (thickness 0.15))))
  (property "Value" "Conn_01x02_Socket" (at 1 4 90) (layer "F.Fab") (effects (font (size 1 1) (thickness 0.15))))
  (pad "1" thru_hole roundrect (at 0 0 270) (size 1.2 1.75) (drill 0.75) (layers "*.Cu" "*.Mask") (remove_unused_layers no)
   (roundrect_rratio 0.208333) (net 8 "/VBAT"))
  (pad "2" thru_hole oval (at 2 0 270) (size 1.2 1.75) (drill 0.75) (layers "*.Cu" "*.Mask") (remove_unused_layers no) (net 5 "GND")))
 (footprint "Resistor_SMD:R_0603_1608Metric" (layer "F.Cu") (at 107.2 91.99)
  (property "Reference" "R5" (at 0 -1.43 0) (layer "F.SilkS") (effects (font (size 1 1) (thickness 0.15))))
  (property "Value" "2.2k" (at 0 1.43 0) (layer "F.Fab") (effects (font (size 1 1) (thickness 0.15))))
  (pad "1" smd roundrect (at -0.825 0) (size 0.8 0.95) (layers "F.Cu" "F.Mask" "F.Paste") (roundrect_rratio 0.25) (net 3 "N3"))
  (pad "2" smd roundrect (at 0.825 0) (size 0.8 0.95) (layers "F.Cu" "F.Mask" "F.Paste") (roundrect_rratio 0.25) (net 51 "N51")))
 (gr_arc (start 103 130) (mid 100.87868 129.12132) (end 100 127) (stroke (width 0.05) (type default)) (locked yes) (layer "Edge.Cuts"))
 (gr_arc (start 185 127) (mid 184.12132 129.12132) (end 182 130) (stroke (width 0.05) (type default)) (locked yes) (layer "Edge.Cuts"))
 (gr_line (start 185 77) (end 185 127) (stroke (width 0.05) (type default)) (locked yes) (layer "Edge.Cuts"))
 (gr_line (start 103 130) (end 182 130) (stroke (width 0.05) (type default)) (locked yes) (layer "Edge.Cuts"))
 (gr_arc (start 182 74) (mid 184.12132 74.87868) (end 185 77) (stroke (width 0.05) (type default)) (locked yes) (layer "Edge.Cuts"))
 (gr_line (start 100 77) (end 100 127) (stroke (width 0.05) (type default)) (locked yes) (layer "Edge.Cuts"))
 (gr_line (start 103 74) (end 182 74) (stroke (width 0.05) (type default)) (locked yes) (layer "Edge.Cuts"))
 (gr_arc (start 100 77) (mid 100.87868 74.87868) (end 103 74) (stroke (width 0.05) (type default)) (locked yes) (layer "Edge.Cuts"))
 (segment (start 130.664999 107.35) (end 125.331802 107.35) (width 0.2) (layer "F.Cu") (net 20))
 (segment (start 125.331802 107.35) (end 116.775 115.906802) (width 0.2) (layer "F.Cu") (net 20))
 (segment (start 131.074999 106.94) (end 130.664999 107.35) (width 0.2) (layer "F.Cu") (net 20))
 (segment (start 116.775 115.906802) (end 116.775 119) (width 0.2) (layer "F.Cu") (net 20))
 (segment (start 132.2 106.94) (end 131.074999 106.94) (width 0.2) (layer "F.Cu") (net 20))
 (segment (start 125.518198 107.8) (end 117.225 116.093198) (width 0.2) (layer "F.Cu") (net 21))
 (segment (start 117.225 116.093198) (end 117.225 119) (width 0.2) (layer "F.Cu") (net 21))
 (segment (start 131.074999 108.21) (end 130.664999 107.8) (width 0.2) (layer "F.Cu") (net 21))
 (segment (start 130.664999 107.8) (end 125.518198 107.8) (width 0.2) (layer "F.Cu") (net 21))
 (segment (start 132.2 108.21) (end 131.074999 108.21) (width 0.2) (layer "F.Cu") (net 21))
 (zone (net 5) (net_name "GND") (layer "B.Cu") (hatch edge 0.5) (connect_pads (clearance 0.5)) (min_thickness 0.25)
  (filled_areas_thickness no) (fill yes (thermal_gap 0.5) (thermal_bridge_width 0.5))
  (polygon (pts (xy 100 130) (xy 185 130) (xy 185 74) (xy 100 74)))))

